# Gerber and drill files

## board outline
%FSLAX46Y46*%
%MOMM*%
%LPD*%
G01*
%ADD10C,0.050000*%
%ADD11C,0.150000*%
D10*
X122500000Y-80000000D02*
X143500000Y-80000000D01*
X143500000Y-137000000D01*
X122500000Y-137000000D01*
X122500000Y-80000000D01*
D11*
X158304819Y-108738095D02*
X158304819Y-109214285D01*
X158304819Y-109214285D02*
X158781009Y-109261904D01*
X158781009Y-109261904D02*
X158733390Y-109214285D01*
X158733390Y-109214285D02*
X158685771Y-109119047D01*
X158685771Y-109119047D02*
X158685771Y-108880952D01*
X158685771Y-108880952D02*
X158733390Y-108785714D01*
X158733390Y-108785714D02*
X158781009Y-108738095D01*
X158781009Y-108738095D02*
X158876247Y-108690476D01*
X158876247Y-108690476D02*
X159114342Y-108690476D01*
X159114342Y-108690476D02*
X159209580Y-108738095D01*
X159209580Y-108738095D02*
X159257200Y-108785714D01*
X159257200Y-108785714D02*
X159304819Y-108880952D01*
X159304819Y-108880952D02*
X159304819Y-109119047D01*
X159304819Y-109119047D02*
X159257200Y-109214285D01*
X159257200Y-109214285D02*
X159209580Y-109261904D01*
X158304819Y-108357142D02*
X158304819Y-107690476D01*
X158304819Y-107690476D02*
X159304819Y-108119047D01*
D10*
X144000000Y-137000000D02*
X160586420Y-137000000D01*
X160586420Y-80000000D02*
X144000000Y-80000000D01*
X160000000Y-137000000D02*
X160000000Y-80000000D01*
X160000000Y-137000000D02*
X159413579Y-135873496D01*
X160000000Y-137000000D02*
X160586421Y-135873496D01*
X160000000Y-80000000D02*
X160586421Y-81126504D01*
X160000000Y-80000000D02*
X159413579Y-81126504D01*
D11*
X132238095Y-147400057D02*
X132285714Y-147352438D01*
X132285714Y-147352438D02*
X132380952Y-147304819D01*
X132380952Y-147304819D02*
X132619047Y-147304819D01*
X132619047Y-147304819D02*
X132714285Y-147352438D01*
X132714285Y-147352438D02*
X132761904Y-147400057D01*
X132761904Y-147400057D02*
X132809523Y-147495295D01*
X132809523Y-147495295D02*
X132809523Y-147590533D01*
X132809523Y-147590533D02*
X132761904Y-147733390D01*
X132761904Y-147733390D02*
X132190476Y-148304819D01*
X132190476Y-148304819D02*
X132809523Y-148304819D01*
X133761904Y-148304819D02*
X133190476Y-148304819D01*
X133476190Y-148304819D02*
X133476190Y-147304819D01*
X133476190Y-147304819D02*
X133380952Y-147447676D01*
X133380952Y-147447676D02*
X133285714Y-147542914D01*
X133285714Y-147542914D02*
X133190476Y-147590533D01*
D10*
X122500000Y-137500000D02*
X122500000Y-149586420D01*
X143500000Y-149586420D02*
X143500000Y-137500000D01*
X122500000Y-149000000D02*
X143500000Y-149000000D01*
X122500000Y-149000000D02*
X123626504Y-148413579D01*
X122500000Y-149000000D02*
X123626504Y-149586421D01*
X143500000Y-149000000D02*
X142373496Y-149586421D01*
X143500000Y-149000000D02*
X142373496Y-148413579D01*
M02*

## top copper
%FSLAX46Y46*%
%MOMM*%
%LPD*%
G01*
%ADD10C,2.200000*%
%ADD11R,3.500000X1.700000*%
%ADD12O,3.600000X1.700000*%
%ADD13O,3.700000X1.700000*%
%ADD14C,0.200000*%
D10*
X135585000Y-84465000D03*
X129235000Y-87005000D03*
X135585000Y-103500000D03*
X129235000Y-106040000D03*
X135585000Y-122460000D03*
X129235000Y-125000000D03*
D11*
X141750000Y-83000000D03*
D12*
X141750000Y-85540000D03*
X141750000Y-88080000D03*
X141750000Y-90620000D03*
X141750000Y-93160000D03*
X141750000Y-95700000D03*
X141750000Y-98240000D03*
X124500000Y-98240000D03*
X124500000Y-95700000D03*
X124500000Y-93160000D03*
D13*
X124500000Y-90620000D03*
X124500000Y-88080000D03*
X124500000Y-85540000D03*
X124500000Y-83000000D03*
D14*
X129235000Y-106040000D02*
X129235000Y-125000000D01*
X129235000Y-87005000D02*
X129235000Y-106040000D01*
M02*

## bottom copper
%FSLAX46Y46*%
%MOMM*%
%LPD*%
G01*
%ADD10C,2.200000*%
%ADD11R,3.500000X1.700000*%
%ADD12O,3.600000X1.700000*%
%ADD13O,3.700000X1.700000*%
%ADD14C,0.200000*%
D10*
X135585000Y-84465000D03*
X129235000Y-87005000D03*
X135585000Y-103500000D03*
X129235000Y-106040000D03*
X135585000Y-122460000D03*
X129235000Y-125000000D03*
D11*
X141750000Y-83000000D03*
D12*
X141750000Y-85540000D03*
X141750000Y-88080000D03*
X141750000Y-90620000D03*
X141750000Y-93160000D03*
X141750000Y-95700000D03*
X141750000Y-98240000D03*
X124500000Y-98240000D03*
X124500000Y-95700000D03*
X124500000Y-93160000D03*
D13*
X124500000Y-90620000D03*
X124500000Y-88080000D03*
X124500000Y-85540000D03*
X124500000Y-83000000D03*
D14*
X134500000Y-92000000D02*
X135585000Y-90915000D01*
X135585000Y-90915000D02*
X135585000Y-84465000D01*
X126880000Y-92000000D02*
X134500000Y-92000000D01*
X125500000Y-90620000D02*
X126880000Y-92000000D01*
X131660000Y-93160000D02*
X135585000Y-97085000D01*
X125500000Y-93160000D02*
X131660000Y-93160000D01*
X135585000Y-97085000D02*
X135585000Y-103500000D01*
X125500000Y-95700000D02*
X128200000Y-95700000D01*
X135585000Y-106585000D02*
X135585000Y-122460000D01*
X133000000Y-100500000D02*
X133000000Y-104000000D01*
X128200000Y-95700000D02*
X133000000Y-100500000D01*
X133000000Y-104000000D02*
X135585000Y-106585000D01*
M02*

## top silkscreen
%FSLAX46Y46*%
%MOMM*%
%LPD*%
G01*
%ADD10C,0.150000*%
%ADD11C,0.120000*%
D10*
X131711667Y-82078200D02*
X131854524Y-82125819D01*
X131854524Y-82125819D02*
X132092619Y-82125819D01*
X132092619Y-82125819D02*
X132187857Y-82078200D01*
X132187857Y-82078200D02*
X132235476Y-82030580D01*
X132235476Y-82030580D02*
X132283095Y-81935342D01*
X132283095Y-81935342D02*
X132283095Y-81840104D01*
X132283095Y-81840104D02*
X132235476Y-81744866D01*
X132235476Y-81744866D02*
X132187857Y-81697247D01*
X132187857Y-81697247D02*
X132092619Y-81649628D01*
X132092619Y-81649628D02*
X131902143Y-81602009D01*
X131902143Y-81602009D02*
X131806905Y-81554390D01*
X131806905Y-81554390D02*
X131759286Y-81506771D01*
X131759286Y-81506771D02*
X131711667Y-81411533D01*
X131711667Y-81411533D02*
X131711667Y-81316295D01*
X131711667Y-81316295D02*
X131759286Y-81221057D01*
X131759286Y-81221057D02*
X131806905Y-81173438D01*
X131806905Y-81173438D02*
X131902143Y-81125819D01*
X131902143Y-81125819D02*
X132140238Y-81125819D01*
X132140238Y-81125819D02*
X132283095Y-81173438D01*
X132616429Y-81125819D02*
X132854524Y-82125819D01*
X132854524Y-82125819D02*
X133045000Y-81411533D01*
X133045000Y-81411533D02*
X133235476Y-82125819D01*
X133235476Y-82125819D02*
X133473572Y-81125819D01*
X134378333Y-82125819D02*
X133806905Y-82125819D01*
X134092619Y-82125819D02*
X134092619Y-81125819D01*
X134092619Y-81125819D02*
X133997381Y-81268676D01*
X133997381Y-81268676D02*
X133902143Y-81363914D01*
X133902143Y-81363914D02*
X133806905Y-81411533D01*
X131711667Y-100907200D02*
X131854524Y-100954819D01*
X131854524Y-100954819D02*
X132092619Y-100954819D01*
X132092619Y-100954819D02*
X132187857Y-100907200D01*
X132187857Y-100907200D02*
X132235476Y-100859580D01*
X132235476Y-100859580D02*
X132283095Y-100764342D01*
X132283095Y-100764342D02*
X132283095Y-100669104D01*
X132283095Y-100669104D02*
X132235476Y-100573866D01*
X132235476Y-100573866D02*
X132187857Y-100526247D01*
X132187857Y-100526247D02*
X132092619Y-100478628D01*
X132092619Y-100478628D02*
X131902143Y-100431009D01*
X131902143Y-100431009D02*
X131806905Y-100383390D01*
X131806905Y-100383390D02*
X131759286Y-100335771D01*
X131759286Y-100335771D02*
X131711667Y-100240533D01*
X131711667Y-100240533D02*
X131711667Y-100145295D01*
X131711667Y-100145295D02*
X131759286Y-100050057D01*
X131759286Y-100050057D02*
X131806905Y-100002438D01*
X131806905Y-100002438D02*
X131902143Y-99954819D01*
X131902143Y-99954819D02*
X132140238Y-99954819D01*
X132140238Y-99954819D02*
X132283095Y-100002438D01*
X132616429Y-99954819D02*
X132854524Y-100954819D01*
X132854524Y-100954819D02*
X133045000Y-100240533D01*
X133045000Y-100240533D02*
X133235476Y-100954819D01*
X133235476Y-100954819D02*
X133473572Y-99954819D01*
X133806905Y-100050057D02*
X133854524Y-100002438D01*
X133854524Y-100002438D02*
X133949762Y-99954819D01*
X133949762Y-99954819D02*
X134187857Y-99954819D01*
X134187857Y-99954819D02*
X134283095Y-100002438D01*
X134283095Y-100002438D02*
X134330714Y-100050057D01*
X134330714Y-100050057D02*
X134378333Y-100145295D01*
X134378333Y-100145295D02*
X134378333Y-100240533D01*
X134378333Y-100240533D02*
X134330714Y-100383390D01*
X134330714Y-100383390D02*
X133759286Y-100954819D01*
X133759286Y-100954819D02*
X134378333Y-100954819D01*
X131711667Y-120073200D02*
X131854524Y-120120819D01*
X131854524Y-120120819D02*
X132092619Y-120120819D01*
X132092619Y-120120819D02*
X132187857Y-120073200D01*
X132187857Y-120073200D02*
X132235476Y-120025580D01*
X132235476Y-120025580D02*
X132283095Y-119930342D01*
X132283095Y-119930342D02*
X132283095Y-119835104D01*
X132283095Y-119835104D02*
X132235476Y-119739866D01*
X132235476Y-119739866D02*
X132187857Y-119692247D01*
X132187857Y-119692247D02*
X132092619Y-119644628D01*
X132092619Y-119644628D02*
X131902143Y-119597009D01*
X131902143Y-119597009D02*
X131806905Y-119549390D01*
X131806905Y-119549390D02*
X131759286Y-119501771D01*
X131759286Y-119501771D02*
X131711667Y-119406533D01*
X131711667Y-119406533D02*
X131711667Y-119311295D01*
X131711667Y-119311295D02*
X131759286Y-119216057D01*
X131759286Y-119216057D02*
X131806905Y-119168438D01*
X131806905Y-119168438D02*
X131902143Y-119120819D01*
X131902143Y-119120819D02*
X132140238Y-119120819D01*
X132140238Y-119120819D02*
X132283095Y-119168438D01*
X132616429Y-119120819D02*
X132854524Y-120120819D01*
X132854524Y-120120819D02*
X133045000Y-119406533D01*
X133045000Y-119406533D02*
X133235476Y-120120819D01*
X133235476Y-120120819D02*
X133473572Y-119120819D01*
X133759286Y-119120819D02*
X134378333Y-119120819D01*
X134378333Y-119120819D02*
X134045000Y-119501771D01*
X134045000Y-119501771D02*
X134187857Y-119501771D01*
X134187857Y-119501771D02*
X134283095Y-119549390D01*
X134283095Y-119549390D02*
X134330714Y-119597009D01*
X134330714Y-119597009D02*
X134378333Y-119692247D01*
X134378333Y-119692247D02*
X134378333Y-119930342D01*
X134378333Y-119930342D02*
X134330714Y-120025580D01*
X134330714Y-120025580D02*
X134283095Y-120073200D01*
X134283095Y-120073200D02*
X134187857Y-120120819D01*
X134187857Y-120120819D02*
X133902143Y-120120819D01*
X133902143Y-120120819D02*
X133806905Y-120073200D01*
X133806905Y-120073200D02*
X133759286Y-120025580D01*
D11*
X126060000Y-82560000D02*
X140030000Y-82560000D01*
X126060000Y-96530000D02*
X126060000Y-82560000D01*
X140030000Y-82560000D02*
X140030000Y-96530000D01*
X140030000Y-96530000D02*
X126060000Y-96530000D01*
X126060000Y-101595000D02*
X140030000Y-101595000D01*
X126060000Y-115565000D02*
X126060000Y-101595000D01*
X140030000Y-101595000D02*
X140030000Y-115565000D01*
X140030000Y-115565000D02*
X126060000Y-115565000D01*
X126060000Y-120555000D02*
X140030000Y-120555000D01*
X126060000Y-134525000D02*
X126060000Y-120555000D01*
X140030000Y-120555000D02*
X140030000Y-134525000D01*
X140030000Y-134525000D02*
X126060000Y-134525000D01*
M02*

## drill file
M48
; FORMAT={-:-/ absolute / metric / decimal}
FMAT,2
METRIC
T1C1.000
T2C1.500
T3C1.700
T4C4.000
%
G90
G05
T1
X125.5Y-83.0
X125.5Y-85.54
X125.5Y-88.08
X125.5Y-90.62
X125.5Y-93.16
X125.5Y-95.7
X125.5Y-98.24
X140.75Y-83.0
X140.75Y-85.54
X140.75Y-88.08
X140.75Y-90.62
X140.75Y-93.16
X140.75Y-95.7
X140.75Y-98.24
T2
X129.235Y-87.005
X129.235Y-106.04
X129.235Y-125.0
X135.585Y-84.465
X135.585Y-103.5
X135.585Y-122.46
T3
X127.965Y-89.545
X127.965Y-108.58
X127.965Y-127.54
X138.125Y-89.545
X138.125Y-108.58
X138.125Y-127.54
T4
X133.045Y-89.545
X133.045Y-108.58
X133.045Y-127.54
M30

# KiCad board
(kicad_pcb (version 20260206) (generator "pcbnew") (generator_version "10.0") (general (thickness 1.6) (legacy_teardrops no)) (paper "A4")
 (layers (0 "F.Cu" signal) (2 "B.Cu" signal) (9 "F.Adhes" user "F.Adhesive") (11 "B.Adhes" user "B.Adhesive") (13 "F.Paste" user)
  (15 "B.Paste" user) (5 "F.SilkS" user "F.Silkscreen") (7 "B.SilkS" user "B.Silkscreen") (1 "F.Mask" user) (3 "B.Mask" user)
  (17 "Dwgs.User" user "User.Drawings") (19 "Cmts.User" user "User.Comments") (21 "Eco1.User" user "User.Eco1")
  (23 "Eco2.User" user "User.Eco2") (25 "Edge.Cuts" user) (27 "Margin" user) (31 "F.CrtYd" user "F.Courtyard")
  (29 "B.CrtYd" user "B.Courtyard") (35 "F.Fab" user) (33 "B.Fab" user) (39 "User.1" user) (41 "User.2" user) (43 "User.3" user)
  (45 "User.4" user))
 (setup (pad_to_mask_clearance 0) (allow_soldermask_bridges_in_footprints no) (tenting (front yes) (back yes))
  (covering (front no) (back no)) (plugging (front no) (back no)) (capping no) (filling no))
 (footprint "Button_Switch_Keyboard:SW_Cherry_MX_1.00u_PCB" (layer "F.Cu") (at 135.585 84.465)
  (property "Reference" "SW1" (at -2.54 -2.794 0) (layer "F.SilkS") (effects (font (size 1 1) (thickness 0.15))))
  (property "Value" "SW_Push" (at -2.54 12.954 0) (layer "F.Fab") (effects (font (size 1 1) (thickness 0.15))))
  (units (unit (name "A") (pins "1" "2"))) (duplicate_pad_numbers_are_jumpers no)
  (fp_line (start -9.525 -1.905) (end 4.445 -1.905) (stroke (width 0.12) (type solid)) (layer "F.SilkS"))
  (fp_line (start -9.525 12.065) (end -9.525 -1.905) (stroke (width 0.12) (type solid)) (layer "F.SilkS"))
  (fp_line (start 4.445 -1.905) (end 4.445 12.065) (stroke (width 0.12) (type solid)) (layer "F.SilkS"))
  (fp_line (start 4.445 12.065) (end -9.525 12.065) (stroke (width 0.12) (type solid)) (layer "F.SilkS"))
  (pad "" np_thru_hole circle (at -7.62 5.08) (size 1.7 1.7) (drill 1.7) (layers "*.Cu" "*.Mask"))
  (pad "" np_thru_hole circle (at -2.54 5.08) (size 4 4) (drill 4) (layers "*.Cu" "*.Mask"))
  (pad "" np_thru_hole circle (at 2.54 5.08) (size 1.7 1.7) (drill 1.7) (layers "*.Cu" "*.Mask"))
  (pad "1" thru_hole circle (at 0 0) (size 2.2 2.2) (drill 1.5) (layers "*.Cu" "*.Mask") (remove_unused_layers no)
   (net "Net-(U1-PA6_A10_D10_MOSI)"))
  (pad "2" thru_hole circle (at -6.35 2.54) (size 2.2 2.2) (drill 1.5) (layers "*.Cu" "*.Mask") (remove_unused_layers no) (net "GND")))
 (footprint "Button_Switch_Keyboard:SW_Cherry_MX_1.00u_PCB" (layer "F.Cu") (at 135.585 103.5)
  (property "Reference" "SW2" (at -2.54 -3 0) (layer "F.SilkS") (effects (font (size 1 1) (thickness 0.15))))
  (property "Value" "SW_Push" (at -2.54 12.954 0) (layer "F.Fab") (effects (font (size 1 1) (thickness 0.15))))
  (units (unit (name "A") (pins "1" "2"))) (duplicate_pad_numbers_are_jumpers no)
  (fp_line (start -9.525 -1.905) (end 4.445 -1.905) (stroke (width 0.12) (type solid)) (layer "F.SilkS"))
  (fp_line (start -9.525 12.065) (end -9.525 -1.905) (stroke (width 0.12) (type solid)) (layer "F.SilkS"))
  (fp_line (start 4.445 -1.905) (end 4.445 12.065) (stroke (width 0.12) (type solid)) (layer "F.SilkS"))
  (fp_line (start 4.445 12.065) (end -9.525 12.065) (stroke (width 0.12) (type solid)) (layer "F.SilkS"))
  (pad "" np_thru_hole circle (at -7.62 5.08) (size 1.7 1.7) (drill 1.7) (layers "*.Cu" "*.Mask"))
  (pad "" np_thru_hole circle (at -2.54 5.08) (size 4 4) (drill 4) (layers "*.Cu" "*.Mask"))
  (pad "" np_thru_hole circle (at 2.54 5.08) (size 1.7 1.7) (drill 1.7) (layers "*.Cu" "*.Mask"))
  (pad "1" thru_hole circle (at 0 0) (size 2.2 2.2) (drill 1.5) (layers "*.Cu" "*.Mask") (remove_unused_layers no)
   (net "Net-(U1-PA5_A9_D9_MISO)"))
  (pad "2" thru_hole circle (at -6.35 2.54) (size 2.2 2.2) (drill 1.5) (layers "*.Cu" "*.Mask") (remove_unused_layers no) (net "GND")))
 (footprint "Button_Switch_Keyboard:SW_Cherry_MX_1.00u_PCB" (layer "F.Cu") (at 135.585 122.46)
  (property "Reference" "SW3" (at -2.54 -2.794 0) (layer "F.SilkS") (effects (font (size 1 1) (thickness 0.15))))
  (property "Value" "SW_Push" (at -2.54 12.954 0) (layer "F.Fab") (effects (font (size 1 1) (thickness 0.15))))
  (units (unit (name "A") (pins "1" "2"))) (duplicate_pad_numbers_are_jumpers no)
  (fp_line (start -9.525 -1.905) (end 4.445 -1.905) (stroke (width 0.12) (type solid)) (layer "F.SilkS"))
  (fp_line (start -9.525 12.065) (end -9.525 -1.905) (stroke (width 0.12) (type solid)) (layer "F.SilkS"))
  (fp_line (start 4.445 -1.905) (end 4.445 12.065) (stroke (width 0.12) (type solid)) (layer "F.SilkS"))
  (fp_line (start 4.445 12.065) (end -9.525 12.065) (stroke (width 0.12) (type solid)) (layer "F.SilkS"))
  (pad "" np_thru_hole circle (at -7.62 5.08) (size 1.7 1.7) (drill 1.7) (layers "*.Cu" "*.Mask"))
  (pad "" np_thru_hole circle (at -2.54 5.08) (size 4 4) (drill 4) (layers "*.Cu" "*.Mask"))
  (pad "" np_thru_hole circle (at 2.54 5.08) (size 1.7 1.7) (drill 1.7) (layers "*.Cu" "*.Mask"))
  (pad "1" thru_hole circle (at 0 0) (size 2.2 2.2) (drill 1.5) (layers "*.Cu" "*.Mask") (remove_unused_layers no)
   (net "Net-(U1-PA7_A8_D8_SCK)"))
  (pad "2" thru_hole circle (at -6.35 2.54) (size 2.2 2.2) (drill 1.5) (layers "*.Cu" "*.Mask") (remove_unused_layers no) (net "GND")))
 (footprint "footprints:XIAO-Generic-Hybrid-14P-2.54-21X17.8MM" (layer "B.Cu") (at 133.125 90.62 180)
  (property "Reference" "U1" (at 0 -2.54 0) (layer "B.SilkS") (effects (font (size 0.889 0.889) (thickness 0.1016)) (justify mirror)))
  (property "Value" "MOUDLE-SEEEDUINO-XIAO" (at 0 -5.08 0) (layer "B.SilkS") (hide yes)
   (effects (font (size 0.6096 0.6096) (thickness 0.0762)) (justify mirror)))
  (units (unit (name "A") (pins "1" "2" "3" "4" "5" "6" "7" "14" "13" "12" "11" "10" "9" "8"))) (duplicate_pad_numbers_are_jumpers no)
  (pad "1" thru_hole rect (at -7.625 7.62 180) (size 3.5 1.7) (drill 1 (offset -1 0)) (layers "*.Cu" "*.Mask") (remove_unused_layers no)
   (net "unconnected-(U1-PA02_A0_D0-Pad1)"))
  (pad "2" thru_hole oval (at -7.625 5.08 180) (size 3.6 1.7) (drill 1 (offset -1 0)) (layers "*.Cu" "*.Mask") (remove_unused_layers no)
   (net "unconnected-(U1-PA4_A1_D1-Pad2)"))
  (pad "3" thru_hole oval (at -7.625 2.54 180) (size 3.6 1.7) (drill 1 (offset -1 0)) (layers "*.Cu" "*.Mask") (remove_unused_layers no)
   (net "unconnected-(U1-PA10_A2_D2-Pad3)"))
  (pad "4" thru_hole oval (at -7.625 0 180) (size 3.6 1.7) (drill 1 (offset -1 0)) (layers "*.Cu" "*.Mask") (remove_unused_layers no)
   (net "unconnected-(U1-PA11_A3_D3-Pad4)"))
  (pad "5" thru_hole oval (at -7.625 -2.54 180) (size 3.6 1.7) (drill 1 (offset -1 0)) (layers "*.Cu" "*.Mask") (remove_unused_layers no)
   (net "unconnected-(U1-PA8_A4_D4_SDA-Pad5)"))
  (pad "6" thru_hole oval (at -7.625 -5.08) (size 3.6 1.7) (drill 1 (offset 1 0)) (layers "*.Cu" "*.Mask") (remove_unused_layers no)
   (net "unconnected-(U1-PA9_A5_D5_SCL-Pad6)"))
  (pad "7" thru_hole oval (at -7.625 -7.62 180) (size 3.6 1.7) (drill 1 (offset -1 0)) (layers "*.Cu" "*.Mask") (remove_unused_layers no)
   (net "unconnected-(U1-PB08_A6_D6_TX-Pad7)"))
  (pad "8" thru_hole oval (at 7.625 -7.62 180) (size 3.6 1.7) (drill 1 (offset 1 0)) (layers "*.Cu" "*.Mask") (remove_unused_layers no)
   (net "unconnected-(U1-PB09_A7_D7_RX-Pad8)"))
  (pad "9" thru_hole oval (at 7.625 -5.08 180) (size 3.6 1.7) (drill 1 (offset 1 0)) (layers "*.Cu" "*.Mask") (remove_unused_layers no)
   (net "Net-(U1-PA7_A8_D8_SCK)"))
  (pad "10" thru_hole oval (at 7.625 -2.54 180) (size 3.6 1.7) (drill 1 (offset 1 0)) (layers "*.Cu" "*.Mask") (remove_unused_layers no)
   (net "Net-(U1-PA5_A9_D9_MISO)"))
  (pad "11" thru_hole oval (at 7.625 0 180) (size 3.7 1.7) (drill 1 (offset 1 0)) (layers "*.Cu" "*.Mask") (remove_unused_layers no)
   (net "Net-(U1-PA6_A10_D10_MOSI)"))
  (pad "12" thru_hole oval (at 7.625 2.54 180) (size 3.7 1.7) (drill 1 (offset 1 0)) (layers "*.Cu" "*.Mask") (remove_unused_layers no)
   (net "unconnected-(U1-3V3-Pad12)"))
  (pad "13" thru_hole oval (at 7.625 5.08 180) (size 3.7 1.7) (drill 1 (offset 1 0)) (layers "*.Cu" "*.Mask") (remove_unused_layers no)
   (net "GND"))
  (pad "14" thru_hole oval (at 7.625 7.62 180) (size 3.7 1.7) (drill 1 (offset 1 0)) (layers "*.Cu" "*.Mask") (remove_unused_layers no)
   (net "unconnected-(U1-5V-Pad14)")))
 (gr_rect (start 122.5 80) (end 143.5 137) (stroke (width 0.05) (type default)) (fill no) (layer "Edge.Cuts"))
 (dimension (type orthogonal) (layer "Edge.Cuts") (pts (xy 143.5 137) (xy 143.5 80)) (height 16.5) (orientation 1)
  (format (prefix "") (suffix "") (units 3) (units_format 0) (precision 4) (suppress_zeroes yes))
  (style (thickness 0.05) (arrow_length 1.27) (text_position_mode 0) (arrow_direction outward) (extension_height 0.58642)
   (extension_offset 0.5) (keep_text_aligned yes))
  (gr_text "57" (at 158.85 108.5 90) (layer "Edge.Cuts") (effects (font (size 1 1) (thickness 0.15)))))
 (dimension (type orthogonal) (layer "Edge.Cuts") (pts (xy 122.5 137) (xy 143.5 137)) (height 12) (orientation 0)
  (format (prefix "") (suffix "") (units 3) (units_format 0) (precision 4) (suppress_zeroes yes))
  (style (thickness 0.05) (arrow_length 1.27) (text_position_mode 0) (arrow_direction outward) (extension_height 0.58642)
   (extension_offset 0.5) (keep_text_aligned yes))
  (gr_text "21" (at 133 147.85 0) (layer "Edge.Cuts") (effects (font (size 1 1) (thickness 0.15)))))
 (segment (start 134.5 92) (end 135.585 90.915) (width 0.2) (layer "B.Cu") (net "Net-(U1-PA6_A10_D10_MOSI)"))
 (segment (start 135.585 90.915) (end 135.585 84.465) (width 0.2) (layer "B.Cu") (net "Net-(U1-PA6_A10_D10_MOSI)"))
 (segment (start 126.88 92) (end 134.5 92) (width 0.2) (layer "B.Cu") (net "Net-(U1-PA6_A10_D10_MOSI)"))
 (segment (start 125.5 90.62) (end 126.88 92) (width 0.2) (layer "B.Cu") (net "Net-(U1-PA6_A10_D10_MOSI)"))
 (segment (start 129.235 106.04) (end 129.235 125) (width 0.2) (layer "F.Cu") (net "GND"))
 (segment (start 129.235 87.005) (end 129.235 106.04) (width 0.2) (layer "F.Cu") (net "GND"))
 (segment (start 131.66 93.16) (end 135.585 97.085) (width 0.2) (layer "B.Cu") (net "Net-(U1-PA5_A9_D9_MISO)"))
 (segment (start 125.5 93.16) (end 131.66 93.16) (width 0.2) (layer "B.Cu") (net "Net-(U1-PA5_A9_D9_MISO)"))
 (segment (start 135.585 97.085) (end 135.585 103.5) (width 0.2) (layer "B.Cu") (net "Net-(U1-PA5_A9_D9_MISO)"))
 (segment (start 125.5 95.7) (end 128.2 95.7) (width 0.2) (layer "B.Cu") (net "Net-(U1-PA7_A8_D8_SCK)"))
 (segment (start 135.585 106.585) (end 135.585 122.46) (width 0.2) (layer "B.Cu") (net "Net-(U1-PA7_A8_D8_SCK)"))
 (segment (start 133 100.5) (end 133 104) (width 0.2) (layer "B.Cu") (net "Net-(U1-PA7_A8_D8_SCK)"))
 (segment (start 128.2 95.7) (end 133 100.5) (width 0.2) (layer "B.Cu") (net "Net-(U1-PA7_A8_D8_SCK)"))
 (segment (start 133 104) (end 135.585 106.585) (width 0.2) (layer "B.Cu") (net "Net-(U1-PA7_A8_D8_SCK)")))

